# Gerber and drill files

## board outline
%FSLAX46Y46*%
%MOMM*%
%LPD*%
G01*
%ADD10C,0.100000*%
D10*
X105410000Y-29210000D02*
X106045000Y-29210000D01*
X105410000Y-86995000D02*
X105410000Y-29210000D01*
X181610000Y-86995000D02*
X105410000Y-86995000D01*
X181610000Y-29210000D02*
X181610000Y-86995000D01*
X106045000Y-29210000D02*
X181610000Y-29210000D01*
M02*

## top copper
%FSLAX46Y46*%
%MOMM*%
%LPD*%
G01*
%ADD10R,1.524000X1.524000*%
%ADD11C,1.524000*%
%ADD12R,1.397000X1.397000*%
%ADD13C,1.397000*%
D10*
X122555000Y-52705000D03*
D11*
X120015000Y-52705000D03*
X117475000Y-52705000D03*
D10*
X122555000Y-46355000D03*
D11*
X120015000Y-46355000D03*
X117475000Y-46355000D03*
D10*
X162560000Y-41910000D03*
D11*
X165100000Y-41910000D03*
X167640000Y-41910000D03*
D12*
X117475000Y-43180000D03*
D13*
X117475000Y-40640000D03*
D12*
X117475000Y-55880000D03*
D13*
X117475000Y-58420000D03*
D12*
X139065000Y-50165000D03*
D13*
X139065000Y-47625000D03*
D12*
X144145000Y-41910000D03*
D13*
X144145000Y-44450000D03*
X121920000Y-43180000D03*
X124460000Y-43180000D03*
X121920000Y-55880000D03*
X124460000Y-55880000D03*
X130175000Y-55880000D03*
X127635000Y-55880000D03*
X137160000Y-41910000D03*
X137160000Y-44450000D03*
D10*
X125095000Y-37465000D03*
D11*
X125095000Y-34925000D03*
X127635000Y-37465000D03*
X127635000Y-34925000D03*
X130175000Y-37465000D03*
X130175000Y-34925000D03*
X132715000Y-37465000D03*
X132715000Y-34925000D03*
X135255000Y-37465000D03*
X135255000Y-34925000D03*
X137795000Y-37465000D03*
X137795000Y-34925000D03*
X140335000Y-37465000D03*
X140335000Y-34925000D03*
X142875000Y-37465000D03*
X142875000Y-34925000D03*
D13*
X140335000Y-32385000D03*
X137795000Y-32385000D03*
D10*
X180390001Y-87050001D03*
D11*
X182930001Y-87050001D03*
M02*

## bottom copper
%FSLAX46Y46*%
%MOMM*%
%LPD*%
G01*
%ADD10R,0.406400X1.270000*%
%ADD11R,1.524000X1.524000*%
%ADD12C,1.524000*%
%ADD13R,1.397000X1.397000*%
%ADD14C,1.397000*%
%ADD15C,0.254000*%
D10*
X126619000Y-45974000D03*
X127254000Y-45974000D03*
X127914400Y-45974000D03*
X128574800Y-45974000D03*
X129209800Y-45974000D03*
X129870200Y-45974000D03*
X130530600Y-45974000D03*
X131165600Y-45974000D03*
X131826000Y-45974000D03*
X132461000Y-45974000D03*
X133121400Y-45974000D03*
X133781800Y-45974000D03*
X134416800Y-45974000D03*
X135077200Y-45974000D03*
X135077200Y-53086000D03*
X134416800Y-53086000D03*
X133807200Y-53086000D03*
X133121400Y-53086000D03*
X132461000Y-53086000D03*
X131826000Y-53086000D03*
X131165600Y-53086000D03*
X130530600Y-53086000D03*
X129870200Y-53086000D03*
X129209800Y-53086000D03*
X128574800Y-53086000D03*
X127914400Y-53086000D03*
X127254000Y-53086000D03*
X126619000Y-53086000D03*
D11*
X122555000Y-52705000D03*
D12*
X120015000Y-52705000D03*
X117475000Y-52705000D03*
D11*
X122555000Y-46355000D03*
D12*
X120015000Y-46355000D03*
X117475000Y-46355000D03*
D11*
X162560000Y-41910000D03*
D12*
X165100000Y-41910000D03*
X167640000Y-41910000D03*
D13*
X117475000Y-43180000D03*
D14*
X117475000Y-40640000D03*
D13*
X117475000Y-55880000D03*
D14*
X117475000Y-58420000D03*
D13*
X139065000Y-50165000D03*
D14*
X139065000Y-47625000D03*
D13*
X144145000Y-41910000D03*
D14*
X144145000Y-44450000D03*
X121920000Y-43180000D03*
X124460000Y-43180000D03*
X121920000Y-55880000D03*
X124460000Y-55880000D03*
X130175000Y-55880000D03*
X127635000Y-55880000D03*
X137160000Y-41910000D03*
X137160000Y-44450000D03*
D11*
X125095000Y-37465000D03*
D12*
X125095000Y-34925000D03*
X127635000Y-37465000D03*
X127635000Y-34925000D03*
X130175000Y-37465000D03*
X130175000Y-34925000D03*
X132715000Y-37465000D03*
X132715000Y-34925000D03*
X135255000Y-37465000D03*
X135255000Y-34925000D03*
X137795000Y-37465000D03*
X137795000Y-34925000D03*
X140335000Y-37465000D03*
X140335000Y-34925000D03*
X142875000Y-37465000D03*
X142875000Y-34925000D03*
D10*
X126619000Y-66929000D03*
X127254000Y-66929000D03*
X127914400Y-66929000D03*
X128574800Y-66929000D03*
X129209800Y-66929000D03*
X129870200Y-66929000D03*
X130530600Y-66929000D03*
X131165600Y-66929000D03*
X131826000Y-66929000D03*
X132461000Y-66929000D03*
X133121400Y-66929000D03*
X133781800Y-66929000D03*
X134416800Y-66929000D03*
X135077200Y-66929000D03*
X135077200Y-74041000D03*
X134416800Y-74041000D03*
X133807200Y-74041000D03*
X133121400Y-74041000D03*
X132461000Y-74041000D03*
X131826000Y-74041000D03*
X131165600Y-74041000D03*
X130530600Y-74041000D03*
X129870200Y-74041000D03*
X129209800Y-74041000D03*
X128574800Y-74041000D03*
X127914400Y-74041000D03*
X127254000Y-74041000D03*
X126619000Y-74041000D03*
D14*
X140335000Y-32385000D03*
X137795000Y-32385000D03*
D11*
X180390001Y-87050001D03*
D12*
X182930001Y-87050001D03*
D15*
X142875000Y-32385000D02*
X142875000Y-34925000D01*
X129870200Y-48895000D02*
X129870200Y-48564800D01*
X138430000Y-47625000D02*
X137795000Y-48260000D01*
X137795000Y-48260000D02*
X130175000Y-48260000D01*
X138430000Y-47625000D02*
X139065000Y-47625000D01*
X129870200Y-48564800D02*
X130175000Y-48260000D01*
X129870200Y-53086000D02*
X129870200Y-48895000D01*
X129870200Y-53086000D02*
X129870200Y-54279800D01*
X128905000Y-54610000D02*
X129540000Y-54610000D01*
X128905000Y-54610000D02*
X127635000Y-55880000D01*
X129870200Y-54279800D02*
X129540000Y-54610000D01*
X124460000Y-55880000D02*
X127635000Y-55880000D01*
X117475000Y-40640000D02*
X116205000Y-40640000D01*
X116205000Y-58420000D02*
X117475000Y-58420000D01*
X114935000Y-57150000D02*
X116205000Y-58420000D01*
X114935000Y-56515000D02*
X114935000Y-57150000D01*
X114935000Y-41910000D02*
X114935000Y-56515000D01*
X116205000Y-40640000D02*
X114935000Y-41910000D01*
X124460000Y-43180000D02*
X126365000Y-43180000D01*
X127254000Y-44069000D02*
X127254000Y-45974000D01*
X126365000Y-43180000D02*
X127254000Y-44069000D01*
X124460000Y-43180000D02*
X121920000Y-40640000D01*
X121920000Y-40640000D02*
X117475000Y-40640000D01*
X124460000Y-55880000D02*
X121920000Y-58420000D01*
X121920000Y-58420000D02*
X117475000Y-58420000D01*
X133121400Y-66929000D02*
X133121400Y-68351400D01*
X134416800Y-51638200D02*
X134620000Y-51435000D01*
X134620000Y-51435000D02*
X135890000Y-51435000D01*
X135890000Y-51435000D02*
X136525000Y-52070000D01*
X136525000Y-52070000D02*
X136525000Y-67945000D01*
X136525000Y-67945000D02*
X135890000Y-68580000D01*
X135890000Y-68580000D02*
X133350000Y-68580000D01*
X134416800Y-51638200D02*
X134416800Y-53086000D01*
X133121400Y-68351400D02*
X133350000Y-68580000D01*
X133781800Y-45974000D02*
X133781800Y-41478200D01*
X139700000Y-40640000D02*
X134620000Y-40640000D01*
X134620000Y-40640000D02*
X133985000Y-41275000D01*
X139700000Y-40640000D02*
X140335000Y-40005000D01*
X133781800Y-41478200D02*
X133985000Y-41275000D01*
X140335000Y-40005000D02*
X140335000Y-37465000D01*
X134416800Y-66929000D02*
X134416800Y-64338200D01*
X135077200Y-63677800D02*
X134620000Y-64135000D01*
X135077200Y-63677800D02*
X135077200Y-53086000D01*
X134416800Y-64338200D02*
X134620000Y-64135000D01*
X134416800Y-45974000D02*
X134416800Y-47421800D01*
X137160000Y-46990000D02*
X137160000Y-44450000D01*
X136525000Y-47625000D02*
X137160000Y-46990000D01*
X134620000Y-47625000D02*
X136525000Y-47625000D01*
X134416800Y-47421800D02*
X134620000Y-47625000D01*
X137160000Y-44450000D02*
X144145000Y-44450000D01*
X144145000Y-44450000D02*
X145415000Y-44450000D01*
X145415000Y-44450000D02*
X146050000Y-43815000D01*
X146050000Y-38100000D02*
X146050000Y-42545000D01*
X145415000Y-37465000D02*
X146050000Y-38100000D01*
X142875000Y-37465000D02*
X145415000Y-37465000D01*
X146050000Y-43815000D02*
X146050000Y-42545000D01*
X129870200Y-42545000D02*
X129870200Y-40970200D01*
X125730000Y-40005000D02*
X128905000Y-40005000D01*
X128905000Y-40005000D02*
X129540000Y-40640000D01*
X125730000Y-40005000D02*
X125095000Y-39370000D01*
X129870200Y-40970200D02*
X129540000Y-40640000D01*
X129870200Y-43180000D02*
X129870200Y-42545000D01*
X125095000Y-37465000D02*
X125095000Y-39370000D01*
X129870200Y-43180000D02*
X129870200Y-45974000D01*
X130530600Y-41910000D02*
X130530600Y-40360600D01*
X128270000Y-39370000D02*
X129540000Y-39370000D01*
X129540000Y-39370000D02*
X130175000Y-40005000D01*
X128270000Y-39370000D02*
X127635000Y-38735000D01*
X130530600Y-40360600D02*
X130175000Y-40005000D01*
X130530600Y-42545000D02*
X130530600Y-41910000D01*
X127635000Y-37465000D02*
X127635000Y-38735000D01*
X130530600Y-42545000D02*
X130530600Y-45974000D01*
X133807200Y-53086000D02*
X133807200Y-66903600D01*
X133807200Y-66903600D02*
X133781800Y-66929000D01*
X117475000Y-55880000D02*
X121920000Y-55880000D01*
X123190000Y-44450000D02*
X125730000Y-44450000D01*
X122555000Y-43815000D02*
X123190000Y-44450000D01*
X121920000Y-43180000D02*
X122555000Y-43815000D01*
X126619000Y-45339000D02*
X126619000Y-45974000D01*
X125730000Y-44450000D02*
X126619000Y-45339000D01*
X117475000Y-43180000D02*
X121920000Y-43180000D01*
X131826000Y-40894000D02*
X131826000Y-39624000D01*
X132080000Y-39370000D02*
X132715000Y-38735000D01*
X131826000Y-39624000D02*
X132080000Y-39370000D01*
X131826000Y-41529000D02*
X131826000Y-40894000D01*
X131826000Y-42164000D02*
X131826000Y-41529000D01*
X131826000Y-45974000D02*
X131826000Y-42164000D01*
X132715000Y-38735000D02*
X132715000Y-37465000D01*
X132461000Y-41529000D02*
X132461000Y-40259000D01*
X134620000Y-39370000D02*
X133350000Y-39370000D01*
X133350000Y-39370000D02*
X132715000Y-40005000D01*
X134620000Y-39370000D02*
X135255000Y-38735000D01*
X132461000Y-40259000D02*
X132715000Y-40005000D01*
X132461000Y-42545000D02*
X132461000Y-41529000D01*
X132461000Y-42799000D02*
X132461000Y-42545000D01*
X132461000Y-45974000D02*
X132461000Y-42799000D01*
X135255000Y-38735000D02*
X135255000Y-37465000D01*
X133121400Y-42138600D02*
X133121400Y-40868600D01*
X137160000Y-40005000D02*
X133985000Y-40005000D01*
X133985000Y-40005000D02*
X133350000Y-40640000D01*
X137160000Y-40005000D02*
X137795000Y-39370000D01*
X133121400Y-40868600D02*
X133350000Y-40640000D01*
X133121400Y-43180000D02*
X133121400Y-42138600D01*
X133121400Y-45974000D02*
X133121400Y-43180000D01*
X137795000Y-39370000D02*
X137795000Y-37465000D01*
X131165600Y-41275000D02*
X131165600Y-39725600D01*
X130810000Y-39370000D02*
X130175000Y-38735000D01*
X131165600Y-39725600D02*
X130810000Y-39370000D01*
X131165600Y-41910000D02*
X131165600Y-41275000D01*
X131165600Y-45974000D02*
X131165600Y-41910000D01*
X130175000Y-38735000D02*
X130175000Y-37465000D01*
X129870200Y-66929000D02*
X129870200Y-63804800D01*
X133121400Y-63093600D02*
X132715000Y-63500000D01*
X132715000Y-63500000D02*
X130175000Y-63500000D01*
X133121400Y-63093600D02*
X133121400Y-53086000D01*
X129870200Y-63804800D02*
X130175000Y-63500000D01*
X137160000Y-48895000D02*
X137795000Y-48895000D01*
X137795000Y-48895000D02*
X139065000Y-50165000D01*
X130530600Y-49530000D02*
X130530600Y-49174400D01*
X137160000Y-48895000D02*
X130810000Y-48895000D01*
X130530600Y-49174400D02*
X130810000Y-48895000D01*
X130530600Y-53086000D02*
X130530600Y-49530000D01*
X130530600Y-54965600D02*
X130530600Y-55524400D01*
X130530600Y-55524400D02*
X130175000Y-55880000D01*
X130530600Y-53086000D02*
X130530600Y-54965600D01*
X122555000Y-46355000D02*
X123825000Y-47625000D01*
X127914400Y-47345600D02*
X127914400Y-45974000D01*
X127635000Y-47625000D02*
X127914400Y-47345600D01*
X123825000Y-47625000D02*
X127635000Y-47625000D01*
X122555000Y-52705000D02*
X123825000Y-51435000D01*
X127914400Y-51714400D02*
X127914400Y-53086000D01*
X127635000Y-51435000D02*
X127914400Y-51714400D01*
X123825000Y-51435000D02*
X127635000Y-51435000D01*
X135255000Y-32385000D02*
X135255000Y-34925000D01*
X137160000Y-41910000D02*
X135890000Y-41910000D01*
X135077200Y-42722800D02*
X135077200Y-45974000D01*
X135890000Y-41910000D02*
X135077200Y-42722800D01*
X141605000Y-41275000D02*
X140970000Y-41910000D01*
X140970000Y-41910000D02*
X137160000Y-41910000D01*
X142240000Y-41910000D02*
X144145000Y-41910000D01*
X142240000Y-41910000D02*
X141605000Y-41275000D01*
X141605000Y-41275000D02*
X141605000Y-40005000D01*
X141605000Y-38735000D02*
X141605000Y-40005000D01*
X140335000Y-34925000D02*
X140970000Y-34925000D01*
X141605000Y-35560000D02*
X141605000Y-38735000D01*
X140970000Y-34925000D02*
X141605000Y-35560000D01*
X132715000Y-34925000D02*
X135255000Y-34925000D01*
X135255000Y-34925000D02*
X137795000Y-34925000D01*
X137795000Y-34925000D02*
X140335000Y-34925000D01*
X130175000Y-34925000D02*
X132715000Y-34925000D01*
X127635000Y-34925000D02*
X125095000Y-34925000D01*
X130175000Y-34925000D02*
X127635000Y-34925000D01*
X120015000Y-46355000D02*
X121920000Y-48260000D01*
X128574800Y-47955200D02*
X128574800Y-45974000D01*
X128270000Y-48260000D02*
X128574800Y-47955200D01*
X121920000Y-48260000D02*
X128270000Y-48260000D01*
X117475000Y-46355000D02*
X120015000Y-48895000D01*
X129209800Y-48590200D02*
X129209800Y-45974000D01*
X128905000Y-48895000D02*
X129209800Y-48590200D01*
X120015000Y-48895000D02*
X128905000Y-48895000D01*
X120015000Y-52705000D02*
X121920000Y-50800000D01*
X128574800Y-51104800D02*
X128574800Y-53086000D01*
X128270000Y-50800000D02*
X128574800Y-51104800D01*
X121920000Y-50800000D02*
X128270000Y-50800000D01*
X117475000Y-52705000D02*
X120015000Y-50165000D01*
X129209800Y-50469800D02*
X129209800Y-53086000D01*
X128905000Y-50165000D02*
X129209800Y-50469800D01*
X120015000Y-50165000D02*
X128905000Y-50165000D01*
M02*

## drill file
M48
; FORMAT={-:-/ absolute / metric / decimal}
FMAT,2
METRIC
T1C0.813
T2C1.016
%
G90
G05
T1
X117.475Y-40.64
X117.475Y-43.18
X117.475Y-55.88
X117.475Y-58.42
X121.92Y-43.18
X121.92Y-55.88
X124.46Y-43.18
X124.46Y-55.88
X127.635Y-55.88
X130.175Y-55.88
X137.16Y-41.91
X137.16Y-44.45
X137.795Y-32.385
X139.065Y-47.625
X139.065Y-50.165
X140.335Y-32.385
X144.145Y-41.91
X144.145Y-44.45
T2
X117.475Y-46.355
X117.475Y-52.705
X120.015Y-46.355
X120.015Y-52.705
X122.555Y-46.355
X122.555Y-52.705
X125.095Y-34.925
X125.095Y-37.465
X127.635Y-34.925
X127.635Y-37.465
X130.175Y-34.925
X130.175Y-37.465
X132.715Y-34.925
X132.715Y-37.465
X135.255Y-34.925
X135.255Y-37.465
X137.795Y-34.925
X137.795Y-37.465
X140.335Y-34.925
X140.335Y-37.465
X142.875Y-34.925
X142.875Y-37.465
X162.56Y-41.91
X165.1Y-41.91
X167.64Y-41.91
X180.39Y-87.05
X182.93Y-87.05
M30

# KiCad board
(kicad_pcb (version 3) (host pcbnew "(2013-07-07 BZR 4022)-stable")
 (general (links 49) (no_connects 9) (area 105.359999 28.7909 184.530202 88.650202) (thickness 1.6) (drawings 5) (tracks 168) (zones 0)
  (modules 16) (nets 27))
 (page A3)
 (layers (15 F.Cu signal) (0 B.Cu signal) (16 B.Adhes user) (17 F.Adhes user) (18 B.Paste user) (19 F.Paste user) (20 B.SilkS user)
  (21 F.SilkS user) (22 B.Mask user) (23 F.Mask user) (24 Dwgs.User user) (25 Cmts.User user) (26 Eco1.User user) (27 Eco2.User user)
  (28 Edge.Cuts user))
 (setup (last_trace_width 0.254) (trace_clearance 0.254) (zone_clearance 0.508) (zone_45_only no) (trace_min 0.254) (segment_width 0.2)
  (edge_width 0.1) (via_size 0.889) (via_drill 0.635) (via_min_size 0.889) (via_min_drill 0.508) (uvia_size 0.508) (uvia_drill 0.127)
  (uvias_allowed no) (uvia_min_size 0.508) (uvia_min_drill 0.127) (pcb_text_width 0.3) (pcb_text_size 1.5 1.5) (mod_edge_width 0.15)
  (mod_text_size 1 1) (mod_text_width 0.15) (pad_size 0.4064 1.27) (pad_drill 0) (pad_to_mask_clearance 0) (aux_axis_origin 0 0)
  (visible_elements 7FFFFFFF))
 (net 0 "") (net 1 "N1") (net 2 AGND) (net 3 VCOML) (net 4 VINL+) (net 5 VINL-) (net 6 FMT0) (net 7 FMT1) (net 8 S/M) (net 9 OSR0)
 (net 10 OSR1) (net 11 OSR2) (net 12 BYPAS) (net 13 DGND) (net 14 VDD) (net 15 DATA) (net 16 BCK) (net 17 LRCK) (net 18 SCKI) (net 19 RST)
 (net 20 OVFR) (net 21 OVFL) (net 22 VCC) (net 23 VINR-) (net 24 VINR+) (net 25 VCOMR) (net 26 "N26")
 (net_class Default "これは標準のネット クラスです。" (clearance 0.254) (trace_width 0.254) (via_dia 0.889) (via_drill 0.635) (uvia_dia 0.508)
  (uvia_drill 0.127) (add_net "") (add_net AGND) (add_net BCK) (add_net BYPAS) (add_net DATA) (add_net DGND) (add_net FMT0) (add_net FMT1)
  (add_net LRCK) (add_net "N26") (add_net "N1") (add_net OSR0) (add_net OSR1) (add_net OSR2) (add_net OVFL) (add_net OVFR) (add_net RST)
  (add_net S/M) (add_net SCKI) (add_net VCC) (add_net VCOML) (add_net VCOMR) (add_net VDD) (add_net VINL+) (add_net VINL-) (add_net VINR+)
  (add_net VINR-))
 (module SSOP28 (layer B.Cu) (at 130.81 49.53)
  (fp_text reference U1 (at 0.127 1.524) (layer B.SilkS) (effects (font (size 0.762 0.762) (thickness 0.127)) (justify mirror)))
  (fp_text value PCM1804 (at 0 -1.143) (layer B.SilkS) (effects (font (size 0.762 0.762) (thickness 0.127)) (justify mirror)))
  (pad 1 smd rect (at -4.191 -3.556) (size 0.4064 1.27) (layers B.Cu B.Paste B.Mask) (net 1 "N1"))
  (pad 2 smd rect (at -3.556 -3.556) (size 0.4064 1.27) (layers B.Cu B.Paste B.Mask) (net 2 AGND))
  (pad 3 smd rect (at -2.8956 -3.556) (size 0.4064 1.27) (layers B.Cu B.Paste B.Mask) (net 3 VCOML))
  (pad 4 smd rect (at -2.2352 -3.556) (size 0.4064 1.27) (layers B.Cu B.Paste B.Mask) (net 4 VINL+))
  (pad 5 smd rect (at -1.6002 -3.556) (size 0.4064 1.27) (layers B.Cu B.Paste B.Mask) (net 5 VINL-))
  (pad 6 smd rect (at -0.9398 -3.556) (size 0.4064 1.27) (layers B.Cu B.Paste B.Mask) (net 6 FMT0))
  (pad 7 smd rect (at -0.2794 -3.556) (size 0.4064 1.27) (layers B.Cu B.Paste B.Mask) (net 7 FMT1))
  (pad 8 smd rect (at 0.3556 -3.556) (size 0.4064 1.27) (layers B.Cu B.Paste B.Mask) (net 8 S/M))
  (pad 9 smd rect (at 1.016 -3.556) (size 0.4064 1.27) (layers B.Cu B.Paste B.Mask) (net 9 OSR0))
  (pad 10 smd rect (at 1.651 -3.556) (size 0.4064 1.27) (layers B.Cu B.Paste B.Mask) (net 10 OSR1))
  (pad 11 smd rect (at 2.3114 -3.556) (size 0.4064 1.27) (layers B.Cu B.Paste B.Mask) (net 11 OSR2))
  (pad 12 smd rect (at 2.9718 -3.556) (size 0.4064 1.27) (layers B.Cu B.Paste B.Mask) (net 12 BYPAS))
  (pad 13 smd rect (at 3.6068 -3.556) (size 0.4064 1.27) (layers B.Cu B.Paste B.Mask) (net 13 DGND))
  (pad 14 smd rect (at 4.2672 -3.556) (size 0.4064 1.27) (layers B.Cu B.Paste B.Mask) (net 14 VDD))
  (pad 15 smd rect (at 4.2672 3.556) (size 0.4064 1.27) (layers B.Cu B.Paste B.Mask) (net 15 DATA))
  (pad 16 smd rect (at 3.6068 3.556) (size 0.4064 1.27) (layers B.Cu B.Paste B.Mask) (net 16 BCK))
  (pad 17 smd rect (at 2.9972 3.556) (size 0.4064 1.27) (layers B.Cu B.Paste B.Mask) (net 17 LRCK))
  (pad 18 smd rect (at 2.3114 3.556) (size 0.4064 1.27) (layers B.Cu B.Paste B.Mask) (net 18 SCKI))
  (pad 19 smd rect (at 1.651 3.556) (size 0.4064 1.27) (layers B.Cu B.Paste B.Mask) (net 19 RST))
  (pad 20 smd rect (at 1.016 3.556) (size 0.4064 1.27) (layers B.Cu B.Paste B.Mask) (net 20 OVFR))
  (pad 21 smd rect (at 0.3556 3.556) (size 0.4064 1.27) (layers B.Cu B.Paste B.Mask) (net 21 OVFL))
  (pad 22 smd rect (at -0.2794 3.556) (size 0.4064 1.27) (layers B.Cu B.Paste B.Mask) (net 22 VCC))
  (pad 23 smd rect (at -0.9398 3.556) (size 0.4064 1.27) (layers B.Cu B.Paste B.Mask) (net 2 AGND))
  (pad 24 smd rect (at -1.6002 3.556) (size 0.4064 1.27) (layers B.Cu B.Paste B.Mask) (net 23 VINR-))
  (pad 25 smd rect (at -2.2352 3.556) (size 0.4064 1.27) (layers B.Cu B.Paste B.Mask) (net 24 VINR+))
  (pad 26 smd rect (at -2.8956 3.556) (size 0.4064 1.27) (layers B.Cu B.Paste B.Mask) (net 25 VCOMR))
  (pad 27 smd rect (at -3.556 3.556) (size 0.4064 1.27) (layers B.Cu B.Paste B.Mask) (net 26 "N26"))
  (pad 28 smd rect (at -4.191 3.556) (size 0.4064 1.27) (layers B.Cu B.Paste B.Mask)))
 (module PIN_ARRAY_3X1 (layer F.Cu) (at 120.015 52.705 180)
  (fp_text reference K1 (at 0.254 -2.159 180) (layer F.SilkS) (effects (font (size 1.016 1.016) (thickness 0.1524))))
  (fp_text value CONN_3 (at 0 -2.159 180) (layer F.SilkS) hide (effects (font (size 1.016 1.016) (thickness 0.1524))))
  (pad 1 thru_hole rect (at -2.54 0 180) (size 1.524 1.524) (drill 1.016) (layers *.Cu *.Mask F.SilkS) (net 25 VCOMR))
  (pad 2 thru_hole circle (at 0 0 180) (size 1.524 1.524) (drill 1.016) (layers *.Cu *.Mask F.SilkS) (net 24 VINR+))
  (pad 3 thru_hole circle (at 2.54 0 180) (size 1.524 1.524) (drill 1.016) (layers *.Cu *.Mask F.SilkS) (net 23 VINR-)))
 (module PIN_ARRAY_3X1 (layer F.Cu) (at 120.015 46.355 180)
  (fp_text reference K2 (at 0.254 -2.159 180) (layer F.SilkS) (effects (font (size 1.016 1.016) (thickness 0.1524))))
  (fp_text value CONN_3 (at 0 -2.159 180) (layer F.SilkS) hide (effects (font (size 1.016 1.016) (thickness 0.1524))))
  (pad 1 thru_hole rect (at -2.54 0 180) (size 1.524 1.524) (drill 1.016) (layers *.Cu *.Mask F.SilkS) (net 3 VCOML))
  (pad 2 thru_hole circle (at 0 0 180) (size 1.524 1.524) (drill 1.016) (layers *.Cu *.Mask F.SilkS) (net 4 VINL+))
  (pad 3 thru_hole circle (at 2.54 0 180) (size 1.524 1.524) (drill 1.016) (layers *.Cu *.Mask F.SilkS) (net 5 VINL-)))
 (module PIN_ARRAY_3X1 (layer F.Cu) (at 165.1 41.91)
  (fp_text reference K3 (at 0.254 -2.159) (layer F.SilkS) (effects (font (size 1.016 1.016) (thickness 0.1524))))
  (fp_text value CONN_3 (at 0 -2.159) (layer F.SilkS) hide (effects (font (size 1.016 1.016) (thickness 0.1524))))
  (pad 1 thru_hole rect (at -2.54 0) (size 1.524 1.524) (drill 1.016) (layers *.Cu *.Mask F.SilkS) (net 21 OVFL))
  (pad 2 thru_hole circle (at 0 0) (size 1.524 1.524) (drill 1.016) (layers *.Cu *.Mask F.SilkS) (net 13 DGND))
  (pad 3 thru_hole circle (at 2.54 0) (size 1.524 1.524) (drill 1.016) (layers *.Cu *.Mask F.SilkS) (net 20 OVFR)))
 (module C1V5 (layer F.Cu) (at 117.475 41.91 90)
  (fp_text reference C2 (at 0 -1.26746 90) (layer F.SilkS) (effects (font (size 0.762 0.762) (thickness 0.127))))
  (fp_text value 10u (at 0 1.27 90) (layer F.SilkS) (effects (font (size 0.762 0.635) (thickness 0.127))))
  (pad 1 thru_hole rect (at -1.27 0 90) (size 1.397 1.397) (drill 0.8128) (layers *.Cu *.Mask F.SilkS) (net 1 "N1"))
  (pad 2 thru_hole circle (at 1.27 0 90) (size 1.397 1.397) (drill 0.8128) (layers *.Cu *.Mask F.SilkS) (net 2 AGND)))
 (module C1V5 (layer F.Cu) (at 117.475 57.15 270)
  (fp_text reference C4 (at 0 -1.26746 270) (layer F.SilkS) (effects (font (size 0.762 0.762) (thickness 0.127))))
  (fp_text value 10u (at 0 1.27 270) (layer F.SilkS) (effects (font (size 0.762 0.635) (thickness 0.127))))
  (pad 1 thru_hole rect (at -1.27 0 270) (size 1.397 1.397) (drill 0.8128) (layers *.Cu *.Mask F.SilkS) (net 26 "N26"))
  (pad 2 thru_hole circle (at 1.27 0 270) (size 1.397 1.397) (drill 0.8128) (layers *.Cu *.Mask F.SilkS) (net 2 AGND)))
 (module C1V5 (layer F.Cu) (at 139.065 48.895 90)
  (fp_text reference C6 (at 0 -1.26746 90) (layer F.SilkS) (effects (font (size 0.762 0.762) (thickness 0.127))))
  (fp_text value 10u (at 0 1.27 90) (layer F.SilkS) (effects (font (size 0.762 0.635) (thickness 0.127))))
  (pad 1 thru_hole rect (at -1.27 0 90) (size 1.397 1.397) (drill 0.8128) (layers *.Cu *.Mask F.SilkS) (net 22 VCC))
  (pad 2 thru_hole circle (at 1.27 0 90) (size 1.397 1.397) (drill 0.8128) (layers *.Cu *.Mask F.SilkS) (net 2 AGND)))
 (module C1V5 (layer F.Cu) (at 144.145 43.18 270)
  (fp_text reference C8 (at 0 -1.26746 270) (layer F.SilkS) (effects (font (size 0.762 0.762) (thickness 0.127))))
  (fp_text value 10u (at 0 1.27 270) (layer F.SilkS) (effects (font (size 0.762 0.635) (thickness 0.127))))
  (pad 1 thru_hole rect (at -1.27 0 270) (size 1.397 1.397) (drill 0.8128) (layers *.Cu *.Mask F.SilkS) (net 14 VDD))
  (pad 2 thru_hole circle (at 1.27 0 270) (size 1.397 1.397) (drill 0.8128) (layers *.Cu *.Mask F.SilkS) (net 13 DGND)))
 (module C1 (layer F.Cu) (at 123.19 43.18)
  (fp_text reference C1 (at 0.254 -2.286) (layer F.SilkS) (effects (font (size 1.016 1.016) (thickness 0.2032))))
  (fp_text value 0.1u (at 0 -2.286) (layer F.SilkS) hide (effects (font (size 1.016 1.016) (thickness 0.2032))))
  (pad 1 thru_hole circle (at -1.27 0) (size 1.397 1.397) (drill 0.8128) (layers *.Cu *.Mask F.SilkS) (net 1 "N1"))
  (pad 2 thru_hole circle (at 1.27 0) (size 1.397 1.397) (drill 0.8128) (layers *.Cu *.Mask F.SilkS) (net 2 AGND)))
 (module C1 (layer F.Cu) (at 123.19 55.88)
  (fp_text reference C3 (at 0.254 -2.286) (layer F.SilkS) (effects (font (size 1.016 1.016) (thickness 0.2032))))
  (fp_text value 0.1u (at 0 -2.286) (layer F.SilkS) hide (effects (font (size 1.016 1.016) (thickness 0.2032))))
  (pad 1 thru_hole circle (at -1.27 0) (size 1.397 1.397) (drill 0.8128) (layers *.Cu *.Mask F.SilkS) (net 26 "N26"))
  (pad 2 thru_hole circle (at 1.27 0) (size 1.397 1.397) (drill 0.8128) (layers *.Cu *.Mask F.SilkS) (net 2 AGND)))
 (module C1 (layer F.Cu) (at 128.905 55.88 180)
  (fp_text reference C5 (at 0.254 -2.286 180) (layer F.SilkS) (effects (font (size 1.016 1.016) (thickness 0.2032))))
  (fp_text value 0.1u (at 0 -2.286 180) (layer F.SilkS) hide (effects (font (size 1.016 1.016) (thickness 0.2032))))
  (pad 1 thru_hole circle (at -1.27 0 180) (size 1.397 1.397) (drill 0.8128) (layers *.Cu *.Mask F.SilkS) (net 22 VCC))
  (pad 2 thru_hole circle (at 1.27 0 180) (size 1.397 1.397) (drill 0.8128) (layers *.Cu *.Mask F.SilkS) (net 2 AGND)))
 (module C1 (layer F.Cu) (at 137.16 43.18 270)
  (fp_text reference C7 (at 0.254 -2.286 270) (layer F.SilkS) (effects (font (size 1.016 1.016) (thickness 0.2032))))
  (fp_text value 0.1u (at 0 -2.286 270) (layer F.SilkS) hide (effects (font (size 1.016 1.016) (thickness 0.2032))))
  (pad 1 thru_hole circle (at -1.27 0 270) (size 1.397 1.397) (drill 0.8128) (layers *.Cu *.Mask F.SilkS) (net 14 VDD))
  (pad 2 thru_hole circle (at 1.27 0 270) (size 1.397 1.397) (drill 0.8128) (layers *.Cu *.Mask F.SilkS) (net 13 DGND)))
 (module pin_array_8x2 (layer F.Cu) (at 133.985 36.195)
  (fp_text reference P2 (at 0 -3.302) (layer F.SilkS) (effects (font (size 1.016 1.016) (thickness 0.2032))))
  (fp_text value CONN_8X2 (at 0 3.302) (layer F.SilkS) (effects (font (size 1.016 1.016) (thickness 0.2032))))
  (pad 1 thru_hole rect (at -8.89 1.27) (size 1.524 1.524) (drill 1.016) (layers *.Cu *.Mask F.SilkS) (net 6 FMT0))
  (pad 2 thru_hole circle (at -8.89 -1.27) (size 1.524 1.524) (drill 1.016) (layers *.Cu *.Mask F.SilkS) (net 14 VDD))
  (pad 3 thru_hole circle (at -6.35 1.27) (size 1.524 1.524) (drill 1.016) (layers *.Cu *.Mask F.SilkS) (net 7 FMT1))
  (pad 4 thru_hole circle (at -6.35 -1.27) (size 1.524 1.524) (drill 1.016) (layers *.Cu *.Mask F.SilkS) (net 14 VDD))
  (pad 5 thru_hole circle (at -3.81 1.27) (size 1.524 1.524) (drill 1.016) (layers *.Cu *.Mask F.SilkS) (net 8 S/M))
  (pad 6 thru_hole circle (at -3.81 -1.27) (size 1.524 1.524) (drill 1.016) (layers *.Cu *.Mask F.SilkS) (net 14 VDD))
  (pad 7 thru_hole circle (at -1.27 1.27) (size 1.524 1.524) (drill 1.016) (layers *.Cu *.Mask F.SilkS) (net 9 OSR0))
  (pad 8 thru_hole circle (at -1.27 -1.27) (size 1.524 1.524) (drill 1.016) (layers *.Cu *.Mask F.SilkS) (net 14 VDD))
  (pad 9 thru_hole circle (at 1.27 1.27) (size 1.524 1.524) (drill 1.016) (layers *.Cu *.Mask F.SilkS) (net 10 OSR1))
  (pad 10 thru_hole circle (at 1.27 -1.27) (size 1.524 1.524) (drill 1.016) (layers *.Cu *.Mask F.SilkS) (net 14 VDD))
  (pad 11 thru_hole circle (at 3.81 1.27) (size 1.524 1.524) (drill 1.016) (layers *.Cu *.Mask F.SilkS) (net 11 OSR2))
  (pad 12 thru_hole circle (at 3.81 -1.27) (size 1.524 1.524) (drill 1.016) (layers *.Cu *.Mask F.SilkS) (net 14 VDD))
  (pad 13 thru_hole circle (at 6.35 1.27) (size 1.524 1.524) (drill 1.016) (layers *.Cu *.Mask F.SilkS) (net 12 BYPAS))
  (pad 14 thru_hole circle (at 6.35 -1.27) (size 1.524 1.524) (drill 1.016) (layers *.Cu *.Mask F.SilkS) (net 14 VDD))
  (pad 15 thru_hole circle (at 8.89 1.27) (size 1.524 1.524) (drill 1.016) (layers *.Cu *.Mask F.SilkS))
  (pad 16 thru_hole circle (at 8.89 -1.27) (size 1.524 1.524) (drill 1.016) (layers *.Cu *.Mask F.SilkS)))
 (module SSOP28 (layer B.Cu) (at 130.81 70.485)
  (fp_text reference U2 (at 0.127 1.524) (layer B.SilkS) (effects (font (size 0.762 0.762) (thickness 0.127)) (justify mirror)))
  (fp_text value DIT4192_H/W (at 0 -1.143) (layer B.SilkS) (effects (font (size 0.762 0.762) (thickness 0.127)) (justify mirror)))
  (pad 1 smd rect (at -4.191 -3.556) (size 0.4064 1.27) (layers B.Cu B.Paste B.Mask))
  (pad 2 smd rect (at -3.556 -3.556) (size 0.4064 1.27) (layers B.Cu B.Paste B.Mask))
  (pad 3 smd rect (at -2.8956 -3.556) (size 0.4064 1.27) (layers B.Cu B.Paste B.Mask))
  (pad 4 smd rect (at -2.2352 -3.556) (size 0.4064 1.27) (layers B.Cu B.Paste B.Mask))
  (pad 5 smd rect (at -1.6002 -3.556) (size 0.4064 1.27) (layers B.Cu B.Paste B.Mask))
  (pad 6 smd rect (at -0.9398 -3.556) (size 0.4064 1.27) (layers B.Cu B.Paste B.Mask) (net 18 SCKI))
  (pad 7 smd rect (at -0.2794 -3.556) (size 0.4064 1.27) (layers B.Cu B.Paste B.Mask))
  (pad 8 smd rect (at 0.3556 -3.556) (size 0.4064 1.27) (layers B.Cu B.Paste B.Mask))
  (pad 9 smd rect (at 1.016 -3.556) (size 0.4064 1.27) (layers B.Cu B.Paste B.Mask))
  (pad 10 smd rect (at 1.651 -3.556) (size 0.4064 1.27) (layers B.Cu B.Paste B.Mask))
  (pad 11 smd rect (at 2.3114 -3.556) (size 0.4064 1.27) (layers B.Cu B.Paste B.Mask) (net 16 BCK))
  (pad 12 smd rect (at 2.9718 -3.556) (size 0.4064 1.27) (layers B.Cu B.Paste B.Mask) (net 17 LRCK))
  (pad 13 smd rect (at 3.6068 -3.556) (size 0.4064 1.27) (layers B.Cu B.Paste B.Mask) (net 15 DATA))
  (pad 14 smd rect (at 4.2672 -3.556) (size 0.4064 1.27) (layers B.Cu B.Paste B.Mask) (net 13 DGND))
  (pad 15 smd rect (at 4.2672 3.556) (size 0.4064 1.27) (layers B.Cu B.Paste B.Mask))
  (pad 16 smd rect (at 3.6068 3.556) (size 0.4064 1.27) (layers B.Cu B.Paste B.Mask))
  (pad 17 smd rect (at 2.9972 3.556) (size 0.4064 1.27) (layers B.Cu B.Paste B.Mask))
  (pad 18 smd rect (at 2.3114 3.556) (size 0.4064 1.27) (layers B.Cu B.Paste B.Mask))
  (pad 19 smd rect (at 1.651 3.556) (size 0.4064 1.27) (layers B.Cu B.Paste B.Mask))
  (pad 20 smd rect (at 1.016 3.556) (size 0.4064 1.27) (layers B.Cu B.Paste B.Mask))
  (pad 21 smd rect (at 0.3556 3.556) (size 0.4064 1.27) (layers B.Cu B.Paste B.Mask))
  (pad 22 smd rect (at -0.2794 3.556) (size 0.4064 1.27) (layers B.Cu B.Paste B.Mask))
  (pad 23 smd rect (at -0.9398 3.556) (size 0.4064 1.27) (layers B.Cu B.Paste B.Mask))
  (pad 24 smd rect (at -1.6002 3.556) (size 0.4064 1.27) (layers B.Cu B.Paste B.Mask))
  (pad 25 smd rect (at -2.2352 3.556) (size 0.4064 1.27) (layers B.Cu B.Paste B.Mask))
  (pad 26 smd rect (at -2.8956 3.556) (size 0.4064 1.27) (layers B.Cu B.Paste B.Mask))
  (pad 27 smd rect (at -3.556 3.556) (size 0.4064 1.27) (layers B.Cu B.Paste B.Mask))
  (pad 28 smd rect (at -4.191 3.556) (size 0.4064 1.27) (layers B.Cu B.Paste B.Mask)))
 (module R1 (layer F.Cu) (at 139.065 32.385 180) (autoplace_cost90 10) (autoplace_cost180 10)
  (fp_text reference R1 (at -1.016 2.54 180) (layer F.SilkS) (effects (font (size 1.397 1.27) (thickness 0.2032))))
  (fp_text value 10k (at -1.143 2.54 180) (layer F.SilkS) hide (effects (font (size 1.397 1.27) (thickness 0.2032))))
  (pad 1 thru_hole circle (at -1.27 0 180) (size 1.397 1.397) (drill 0.8128) (layers *.Cu *.Mask F.SilkS) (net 19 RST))
  (pad 2 thru_hole circle (at 1.27 0 180) (size 1.397 1.397) (drill 0.8128) (layers *.Cu *.Mask F.SilkS) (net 14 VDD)))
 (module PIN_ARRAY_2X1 (layer F.Cu) (at 181.660001 87.050001)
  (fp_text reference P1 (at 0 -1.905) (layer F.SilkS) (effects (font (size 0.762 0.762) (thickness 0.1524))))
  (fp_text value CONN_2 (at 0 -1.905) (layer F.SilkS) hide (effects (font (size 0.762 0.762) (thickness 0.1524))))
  (pad 1 thru_hole rect (at -1.27 0) (size 1.524 1.524) (drill 1.016) (layers *.Cu *.Mask F.SilkS) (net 19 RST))
  (pad 2 thru_hole circle (at 1.27 0) (size 1.524 1.524) (drill 1.016) (layers *.Cu *.Mask F.SilkS) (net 13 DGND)))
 (gr_line (start 105.41 29.21) (end 106.045 29.21) (angle 90) (layer Edge.Cuts) (width 0.1))
 (gr_line (start 105.41 86.995) (end 105.41 29.21) (angle 90) (layer Edge.Cuts) (width 0.1))
 (gr_line (start 181.61 86.995) (end 105.41 86.995) (angle 90) (layer Edge.Cuts) (width 0.1))
 (gr_line (start 181.61 29.21) (end 181.61 86.995) (angle 90) (layer Edge.Cuts) (width 0.1))
 (gr_line (start 106.045 29.21) (end 181.61 29.21) (angle 90) (layer Edge.Cuts) (width 0.1))
 (segment (start 142.875 32.385) (end 142.875 34.925) (width 0.254) (layer B.Cu) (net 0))
 (segment (start 129.8702 48.895) (end 129.8702 48.5648) (width 0.254) (layer B.Cu) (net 2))
 (segment (start 138.43 47.625) (end 137.795 48.26) (width 0.254) (layer B.Cu) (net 2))
 (segment (start 137.795 48.26) (end 130.175 48.26) (width 0.254) (layer B.Cu) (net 2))
 (segment (start 138.43 47.625) (end 139.065 47.625) (width 0.254) (layer B.Cu) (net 2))
 (segment (start 129.8702 48.5648) (end 130.175 48.26) (width 0.254) (layer B.Cu) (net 2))
 (segment (start 129.8702 53.086) (end 129.8702 48.895) (width 0.254) (layer B.Cu) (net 2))
 (segment (start 129.8702 53.086) (end 129.8702 54.2798) (width 0.254) (layer B.Cu) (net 2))
 (segment (start 128.905 54.61) (end 129.54 54.61) (width 0.254) (layer B.Cu) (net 2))
 (segment (start 128.905 54.61) (end 127.635 55.88) (width 0.254) (layer B.Cu) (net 2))
 (segment (start 129.8702 54.2798) (end 129.54 54.61) (width 0.254) (layer B.Cu) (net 2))
 (segment (start 124.46 55.88) (end 127.635 55.88) (width 0.254) (layer B.Cu) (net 2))
 (segment (start 117.475 40.64) (end 116.205 40.64) (width 0.254) (layer B.Cu) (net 2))
 (segment (start 116.205 58.42) (end 117.475 58.42) (width 0.254) (layer B.Cu) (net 2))
 (segment (start 114.935 57.15) (end 116.205 58.42) (width 0.254) (layer B.Cu) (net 2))
 (segment (start 114.935 56.515) (end 114.935 57.15) (width 0.254) (layer B.Cu) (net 2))
 (segment (start 114.935 41.91) (end 114.935 56.515) (width 0.254) (layer B.Cu) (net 2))
 (segment (start 116.205 40.64) (end 114.935 41.91) (width 0.254) (layer B.Cu) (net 2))
 (segment (start 124.46 43.18) (end 126.365 43.18) (width 0.254) (layer B.Cu) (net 2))
 (segment (start 127.254 44.069) (end 127.254 45.974) (width 0.254) (layer B.Cu) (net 2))
 (segment (start 126.365 43.18) (end 127.254 44.069) (width 0.254) (layer B.Cu) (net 2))
 (segment (start 124.46 43.18) (end 121.92 40.64) (width 0.254) (layer B.Cu) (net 2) (status 80000))
 (segment (start 121.92 40.64) (end 117.475 40.64) (width 0.254) (layer B.Cu) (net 2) (status 80000))
 (segment (start 124.46 55.88) (end 121.92 58.42) (width 0.254) (layer B.Cu) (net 2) (status 80000))
 (segment (start 121.92 58.42) (end 117.475 58.42) (width 0.254) (layer B.Cu) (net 2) (status 80000))
 (segment (start 133.1214 66.929) (end 133.1214 68.3514) (width 0.254) (layer B.Cu) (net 16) (status 400000))
 (segment (start 134.4168 51.6382) (end 134.62 51.435) (width 0.254) (layer B.Cu) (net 16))
 (segment (start 134.62 51.435) (end 135.89 51.435) (width 0.254) (layer B.Cu) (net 16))
 (segment (start 135.89 51.435) (end 136.525 52.07) (width 0.254) (layer B.Cu) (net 16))
 (segment (start 136.525 52.07) (end 136.525 67.945) (width 0.254) (layer B.Cu) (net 16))
 (segment (start 136.525 67.945) (end 135.89 68.58) (width 0.254) (layer B.Cu) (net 16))
 (segment (start 135.89 68.58) (end 133.35 68.58) (width 0.254) (layer B.Cu) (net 16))
 (segment (start 134.4168 51.6382) (end 134.4168 53.086) (width 0.254) (layer B.Cu) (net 16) (status 800000))
 (segment (start 133.1214 68.3514) (end 133.35 68.58) (width 0.254) (layer B.Cu) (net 16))
 (segment (start 133.7818 45.974) (end 133.7818 41.4782) (width 0.254) (layer B.Cu) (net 12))
 (segment (start 139.7 40.64) (end 134.62 40.64) (width 0.254) (layer B.Cu) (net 12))
 (segment (start 134.62 40.64) (end 133.985 41.275) (width 0.254) (layer B.Cu) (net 12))
 (segment (start 139.7 40.64) (end 140.335 40.005) (width 0.254) (layer B.Cu) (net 12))
 (segment (start 133.7818 41.4782) (end 133.985 41.275) (width 0.254) (layer B.Cu) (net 12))
 (segment (start 140.335 40.005) (end 140.335 37.465) (width 0.254) (layer B.Cu) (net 12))
 (segment (start 134.4168 66.929) (end 134.4168 64.3382) (width 0.254) (layer B.Cu) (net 15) (status 400000))
 (segment (start 135.0772 63.6778) (end 134.62 64.135) (width 0.254) (layer B.Cu) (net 15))
 (segment (start 135.0772 63.6778) (end 135.0772 53.086) (width 0.254) (layer B.Cu) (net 15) (status 800000))
 (segment (start 134.4168 64.3382) (end 134.62 64.135) (width 0.254) (layer B.Cu) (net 15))
 (segment (start 134.4168 45.974) (end 134.4168 47.4218) (width 0.254) (layer B.Cu) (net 13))
 (segment (start 137.16 46.99) (end 137.16 44.45) (width 0.254) (layer B.Cu) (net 13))
 (segment (start 136.525 47.625) (end 137.16 46.99) (width 0.254) (layer B.Cu) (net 13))
 (segment (start 134.62 47.625) (end 136.525 47.625) (width 0.254) (layer B.Cu) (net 13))
 (segment (start 134.4168 47.4218) (end 134.62 47.625) (width 0.254) (layer B.Cu) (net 13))
 (segment (start 137.16 44.45) (end 144.145 44.45) (width 0.254) (layer B.Cu) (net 13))
 (segment (start 144.145 44.45) (end 145.415 44.45) (width 0.254) (layer B.Cu) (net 13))
 (segment (start 145.415 44.45) (end 146.05 43.815) (width 0.254) (layer B.Cu) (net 13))
 (segment (start 146.05 38.1) (end 146.05 42.545) (width 0.254) (layer B.Cu) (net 13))
 (segment (start 145.415 37.465) (end 146.05 38.1) (width 0.254) (layer B.Cu) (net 13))
 (segment (start 142.875 37.465) (end 145.415 37.465) (width 0.254) (layer B.Cu) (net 13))
 (segment (start 146.05 43.815) (end 146.05 42.545) (width 0.254) (layer B.Cu) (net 13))
 (segment (start 129.8702 42.545) (end 129.8702 40.9702) (width 0.254) (layer B.Cu) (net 6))
 (segment (start 125.73 40.005) (end 128.905 40.005) (width 0.254) (layer B.Cu) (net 6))
 (segment (start 128.905 40.005) (end 129.54 40.64) (width 0.254) (layer B.Cu) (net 6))
 (segment (start 125.73 40.005) (end 125.095 39.37) (width 0.254) (layer B.Cu) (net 6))
 (segment (start 129.8702 40.9702) (end 129.54 40.64) (width 0.254) (layer B.Cu) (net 6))
 (segment (start 129.8702 43.18) (end 129.8702 42.545) (width 0.254) (layer B.Cu) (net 6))
 (segment (start 125.095 37.465) (end 125.095 39.37) (width 0.254) (layer B.Cu) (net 6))
 (segment (start 129.8702 43.18) (end 129.8702 45.974) (width 0.254) (layer B.Cu) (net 6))
 (segment (start 130.5306 41.91) (end 130.5306 40.3606) (width 0.254) (layer B.Cu) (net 7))
 (segment (start 128.27 39.37) (end 129.54 39.37) (width 0.254) (layer B.Cu) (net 7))
 (segment (start 129.54 39.37) (end 130.175 40.005) (width 0.254) (layer B.Cu) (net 7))
 (segment (start 128.27 39.37) (end 127.635 38.735) (width 0.254) (layer B.Cu) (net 7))
 (segment (start 130.5306 40.3606) (end 130.175 40.005) (width 0.254) (layer B.Cu) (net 7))
 (segment (start 130.5306 42.545) (end 130.5306 41.91) (width 0.254) (layer B.Cu) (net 7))
 (segment (start 127.635 37.465) (end 127.635 38.735) (width 0.254) (layer B.Cu) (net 7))
 (segment (start 130.5306 42.545) (end 130.5306 45.974) (width 0.254) (layer B.Cu) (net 7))
 (segment (start 133.8072 53.086) (end 133.8072 66.9036) (width 0.254) (layer B.Cu) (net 17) (status C00000))
 (segment (start 133.8072 66.9036) (end 133.7818 66.929) (width 0.254) (layer B.Cu) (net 17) (status C00000))
 (segment (start 117.475 55.88) (end 121.92 55.88) (width 0.254) (layer B.Cu) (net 26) (status 80000))
 (segment (start 123.19 44.45) (end 125.73 44.45) (width 0.254) (layer B.Cu) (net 1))
 (segment (start 122.555 43.815) (end 123.19 44.45) (width 0.254) (layer B.Cu) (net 1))
 (segment (start 121.92 43.18) (end 122.555 43.815) (width 0.254) (layer B.Cu) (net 1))
 (segment (start 126.619 45.339) (end 126.619 45.974) (width 0.254) (layer B.Cu) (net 1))
 (segment (start 125.73 44.45) (end 126.619 45.339) (width 0.254) (layer B.Cu) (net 1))
 (segment (start 117.475 43.18) (end 121.92 43.18) (width 0.254) (layer B.Cu) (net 1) (status 80000))
 (segment (start 131.826 40.894) (end 131.826 39.624) (width 0.254) (layer B.Cu) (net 9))
 (segment (start 132.08 39.37) (end 132.715 38.735) (width 0.254) (layer B.Cu) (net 9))
 (segment (start 131.826 39.624) (end 132.08 39.37) (width 0.254) (layer B.Cu) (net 9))
 (segment (start 131.826 41.529) (end 131.826 40.894) (width 0.254) (layer B.Cu) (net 9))
 (segment (start 131.826 42.164) (end 131.826 41.529) (width 0.254) (layer B.Cu) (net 9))
 (segment (start 131.826 45.974) (end 131.826 42.164) (width 0.254) (layer B.Cu) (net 9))
 (segment (start 132.715 38.735) (end 132.715 37.465) (width 0.254) (layer B.Cu) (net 9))
 (segment (start 132.461 41.529) (end 132.461 40.259) (width 0.254) (layer B.Cu) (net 10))
 (segment (start 134.62 39.37) (end 133.35 39.37) (width 0.254) (layer B.Cu) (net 10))
 (segment (start 133.35 39.37) (end 132.715 40.005) (width 0.254) (layer B.Cu) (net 10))
 (segment (start 134.62 39.37) (end 135.255 38.735) (width 0.254) (layer B.Cu) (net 10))
 (segment (start 132.461 40.259) (end 132.715 40.005) (width 0.254) (layer B.Cu) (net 10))
 (segment (start 132.461 42.545) (end 132.461 41.529) (width 0.254) (layer B.Cu) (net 10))
 (segment (start 132.461 42.799) (end 132.461 42.545) (width 0.254) (layer B.Cu) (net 10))
 (segment (start 132.461 45.974) (end 132.461 42.799) (width 0.254) (layer B.Cu) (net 10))
 (segment (start 135.255 38.735) (end 135.255 37.465) (width 0.254) (layer B.Cu) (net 10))
 (segment (start 133.1214 42.1386) (end 133.1214 40.8686) (width 0.254) (layer B.Cu) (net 11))
 (segment (start 137.16 40.005) (end 133.985 40.005) (width 0.254) (layer B.Cu) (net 11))
 (segment (start 133.985 40.005) (end 133.35 40.64) (width 0.254) (layer B.Cu) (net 11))
 (segment (start 137.16 40.005) (end 137.795 39.37) (width 0.254) (layer B.Cu) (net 11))
 (segment (start 133.1214 40.8686) (end 133.35 40.64) (width 0.254) (layer B.Cu) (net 11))
 (segment (start 133.1214 43.18) (end 133.1214 42.1386) (width 0.254) (layer B.Cu) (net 11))
 (segment (start 133.1214 45.974) (end 133.1214 43.18) (width 0.254) (layer B.Cu) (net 11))
 (segment (start 137.795 39.37) (end 137.795 37.465) (width 0.254) (layer B.Cu) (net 11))
 (segment (start 131.1656 41.275) (end 131.1656 39.7256) (width 0.254) (layer B.Cu) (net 8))
 (segment (start 130.81 39.37) (end 130.175 38.735) (width 0.254) (layer B.Cu) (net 8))
 (segment (start 131.1656 39.7256) (end 130.81 39.37) (width 0.254) (layer B.Cu) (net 8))
 (segment (start 131.1656 41.91) (end 131.1656 41.275) (width 0.254) (layer B.Cu) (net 8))
 (segment (start 131.1656 45.974) (end 131.1656 41.91) (width 0.254) (layer B.Cu) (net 8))
 (segment (start 130.175 38.735) (end 130.175 37.465) (width 0.254) (layer B.Cu) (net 8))
 (segment (start 129.8702 66.929) (end 129.8702 63.8048) (width 0.254) (layer B.Cu) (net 18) (status 400000))
 (segment (start 133.1214 63.0936) (end 132.715 63.5) (width 0.254) (layer B.Cu) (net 18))
 (segment (start 132.715 63.5) (end 130.175 63.5) (width 0.254) (layer B.Cu) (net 18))
 (segment (start 133.1214 63.0936) (end 133.1214 53.086) (width 0.254) (layer B.Cu) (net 18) (status 800000))
 (segment (start 129.8702 63.8048) (end 130.175 63.5) (width 0.254) (layer B.Cu) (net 18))
 (segment (start 137.16 48.895) (end 137.795 48.895) (width 0.254) (layer B.Cu) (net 22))
 (segment (start 137.795 48.895) (end 139.065 50.165) (width 0.254) (layer B.Cu) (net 22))
 (segment (start 130.5306 49.53) (end 130.5306 49.1744) (width 0.254) (layer B.Cu) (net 22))
 (segment (start 137.16 48.895) (end 130.81 48.895) (width 0.254) (layer B.Cu) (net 22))
 (segment (start 130.5306 49.1744) (end 130.81 48.895) (width 0.254) (layer B.Cu) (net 22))
 (segment (start 130.5306 53.086) (end 130.5306 49.53) (width 0.254) (layer B.Cu) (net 22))
 (segment (start 130.5306 54.9656) (end 130.5306 55.5244) (width 0.254) (layer B.Cu) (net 22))
 (segment (start 130.5306 55.5244) (end 130.175 55.88) (width 0.254) (layer B.Cu) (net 22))
 (segment (start 130.5306 53.086) (end 130.5306 54.9656) (width 0.254) (layer B.Cu) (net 22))
 (segment (start 122.555 46.355) (end 123.825 47.625) (width 0.254) (layer B.Cu) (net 3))
 (segment (start 127.9144 47.3456) (end 127.9144 45.974) (width 0.254) (layer B.Cu) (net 3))
 (segment (start 127.635 47.625) (end 127.9144 47.3456) (width 0.254) (layer B.Cu) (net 3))
 (segment (start 123.825 47.625) (end 127.635 47.625) (width 0.254) (layer B.Cu) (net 3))
 (segment (start 122.555 52.705) (end 123.825 51.435) (width 0.254) (layer B.Cu) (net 25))
 (segment (start 127.9144 51.7144) (end 127.9144 53.086) (width 0.254) (layer B.Cu) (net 25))
 (segment (start 127.635 51.435) (end 127.9144 51.7144) (width 0.254) (layer B.Cu) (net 25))
 (segment (start 123.825 51.435) (end 127.635 51.435) (width 0.254) (layer B.Cu) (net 25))
 (segment (start 135.255 32.385) (end 135.255 34.925) (width 0.254) (layer B.Cu) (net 14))
 (segment (start 137.16 41.91) (end 135.89 41.91) (width 0.254) (layer B.Cu) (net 14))
 (segment (start 135.0772 42.7228) (end 135.0772 45.974) (width 0.254) (layer B.Cu) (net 14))
 (segment (start 135.89 41.91) (end 135.0772 42.7228) (width 0.254) (layer B.Cu) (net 14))
 (segment (start 141.605 41.275) (end 140.97 41.91) (width 0.254) (layer B.Cu) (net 14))
 (segment (start 140.97 41.91) (end 137.16 41.91) (width 0.254) (layer B.Cu) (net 14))
 (segment (start 142.24 41.91) (end 144.145 41.91) (width 0.254) (layer B.Cu) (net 14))
 (segment (start 142.24 41.91) (end 141.605 41.275) (width 0.254) (layer B.Cu) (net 14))
 (segment (start 141.605 41.275) (end 141.605 40.005) (width 0.254) (layer B.Cu) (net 14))
 (segment (start 141.605 38.735) (end 141.605 40.005) (width 0.254) (layer B.Cu) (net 14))
 (segment (start 140.335 34.925) (end 140.97 34.925) (width 0.254) (layer B.Cu) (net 14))
 (segment (start 141.605 35.56) (end 141.605 38.735) (width 0.254) (layer B.Cu) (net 14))
 (segment (start 140.97 34.925) (end 141.605 35.56) (width 0.254) (layer B.Cu) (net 14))
 (segment (start 132.715 34.925) (end 135.255 34.925) (width 0.254) (layer B.Cu) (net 14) (status 80000))
 (segment (start 135.255 34.925) (end 137.795 34.925) (width 0.254) (layer B.Cu) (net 14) (status 80000))
 (segment (start 137.795 34.925) (end 140.335 34.925) (width 0.254) (layer B.Cu) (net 14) (status 80000))
 (segment (start 130.175 34.925) (end 132.715 34.925) (width 0.254) (layer B.Cu) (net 14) (status 80000))
 (segment (start 127.635 34.925) (end 125.095 34.925) (width 0.254) (layer B.Cu) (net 14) (status 80000))
 (segment (start 130.175 34.925) (end 127.635 34.925) (width 0.254) (layer B.Cu) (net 14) (status 80000))
 (segment (start 120.015 46.355) (end 121.92 48.26) (width 0.254) (layer B.Cu) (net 4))
 (segment (start 128.5748 47.9552) (end 128.5748 45.974) (width 0.254) (layer B.Cu) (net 4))
 (segment (start 128.27 48.26) (end 128.5748 47.9552) (width 0.254) (layer B.Cu) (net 4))
 (segment (start 121.92 48.26) (end 128.27 48.26) (width 0.254) (layer B.Cu) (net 4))
 (segment (start 117.475 46.355) (end 120.015 48.895) (width 0.254) (layer B.Cu) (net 5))
 (segment (start 129.2098 48.5902) (end 129.2098 45.974) (width 0.254) (layer B.Cu) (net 5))
 (segment (start 128.905 48.895) (end 129.2098 48.5902) (width 0.254) (layer B.Cu) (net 5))
 (segment (start 120.015 48.895) (end 128.905 48.895) (width 0.254) (layer B.Cu) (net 5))
 (segment (start 120.015 52.705) (end 121.92 50.8) (width 0.254) (layer B.Cu) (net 24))
 (segment (start 128.5748 51.1048) (end 128.5748 53.086) (width 0.254) (layer B.Cu) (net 24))
 (segment (start 128.27 50.8) (end 128.5748 51.1048) (width 0.254) (layer B.Cu) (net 24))
 (segment (start 121.92 50.8) (end 128.27 50.8) (width 0.254) (layer B.Cu) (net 24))
 (segment (start 117.475 52.705) (end 120.015 50.165) (width 0.254) (layer B.Cu) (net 23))
 (segment (start 129.2098 50.4698) (end 129.2098 53.086) (width 0.254) (layer B.Cu) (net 23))
 (segment (start 128.905 50.165) (end 129.2098 50.4698) (width 0.254) (layer B.Cu) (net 23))
 (segment (start 120.015 50.165) (end 128.905 50.165) (width 0.254) (layer B.Cu) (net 23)))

